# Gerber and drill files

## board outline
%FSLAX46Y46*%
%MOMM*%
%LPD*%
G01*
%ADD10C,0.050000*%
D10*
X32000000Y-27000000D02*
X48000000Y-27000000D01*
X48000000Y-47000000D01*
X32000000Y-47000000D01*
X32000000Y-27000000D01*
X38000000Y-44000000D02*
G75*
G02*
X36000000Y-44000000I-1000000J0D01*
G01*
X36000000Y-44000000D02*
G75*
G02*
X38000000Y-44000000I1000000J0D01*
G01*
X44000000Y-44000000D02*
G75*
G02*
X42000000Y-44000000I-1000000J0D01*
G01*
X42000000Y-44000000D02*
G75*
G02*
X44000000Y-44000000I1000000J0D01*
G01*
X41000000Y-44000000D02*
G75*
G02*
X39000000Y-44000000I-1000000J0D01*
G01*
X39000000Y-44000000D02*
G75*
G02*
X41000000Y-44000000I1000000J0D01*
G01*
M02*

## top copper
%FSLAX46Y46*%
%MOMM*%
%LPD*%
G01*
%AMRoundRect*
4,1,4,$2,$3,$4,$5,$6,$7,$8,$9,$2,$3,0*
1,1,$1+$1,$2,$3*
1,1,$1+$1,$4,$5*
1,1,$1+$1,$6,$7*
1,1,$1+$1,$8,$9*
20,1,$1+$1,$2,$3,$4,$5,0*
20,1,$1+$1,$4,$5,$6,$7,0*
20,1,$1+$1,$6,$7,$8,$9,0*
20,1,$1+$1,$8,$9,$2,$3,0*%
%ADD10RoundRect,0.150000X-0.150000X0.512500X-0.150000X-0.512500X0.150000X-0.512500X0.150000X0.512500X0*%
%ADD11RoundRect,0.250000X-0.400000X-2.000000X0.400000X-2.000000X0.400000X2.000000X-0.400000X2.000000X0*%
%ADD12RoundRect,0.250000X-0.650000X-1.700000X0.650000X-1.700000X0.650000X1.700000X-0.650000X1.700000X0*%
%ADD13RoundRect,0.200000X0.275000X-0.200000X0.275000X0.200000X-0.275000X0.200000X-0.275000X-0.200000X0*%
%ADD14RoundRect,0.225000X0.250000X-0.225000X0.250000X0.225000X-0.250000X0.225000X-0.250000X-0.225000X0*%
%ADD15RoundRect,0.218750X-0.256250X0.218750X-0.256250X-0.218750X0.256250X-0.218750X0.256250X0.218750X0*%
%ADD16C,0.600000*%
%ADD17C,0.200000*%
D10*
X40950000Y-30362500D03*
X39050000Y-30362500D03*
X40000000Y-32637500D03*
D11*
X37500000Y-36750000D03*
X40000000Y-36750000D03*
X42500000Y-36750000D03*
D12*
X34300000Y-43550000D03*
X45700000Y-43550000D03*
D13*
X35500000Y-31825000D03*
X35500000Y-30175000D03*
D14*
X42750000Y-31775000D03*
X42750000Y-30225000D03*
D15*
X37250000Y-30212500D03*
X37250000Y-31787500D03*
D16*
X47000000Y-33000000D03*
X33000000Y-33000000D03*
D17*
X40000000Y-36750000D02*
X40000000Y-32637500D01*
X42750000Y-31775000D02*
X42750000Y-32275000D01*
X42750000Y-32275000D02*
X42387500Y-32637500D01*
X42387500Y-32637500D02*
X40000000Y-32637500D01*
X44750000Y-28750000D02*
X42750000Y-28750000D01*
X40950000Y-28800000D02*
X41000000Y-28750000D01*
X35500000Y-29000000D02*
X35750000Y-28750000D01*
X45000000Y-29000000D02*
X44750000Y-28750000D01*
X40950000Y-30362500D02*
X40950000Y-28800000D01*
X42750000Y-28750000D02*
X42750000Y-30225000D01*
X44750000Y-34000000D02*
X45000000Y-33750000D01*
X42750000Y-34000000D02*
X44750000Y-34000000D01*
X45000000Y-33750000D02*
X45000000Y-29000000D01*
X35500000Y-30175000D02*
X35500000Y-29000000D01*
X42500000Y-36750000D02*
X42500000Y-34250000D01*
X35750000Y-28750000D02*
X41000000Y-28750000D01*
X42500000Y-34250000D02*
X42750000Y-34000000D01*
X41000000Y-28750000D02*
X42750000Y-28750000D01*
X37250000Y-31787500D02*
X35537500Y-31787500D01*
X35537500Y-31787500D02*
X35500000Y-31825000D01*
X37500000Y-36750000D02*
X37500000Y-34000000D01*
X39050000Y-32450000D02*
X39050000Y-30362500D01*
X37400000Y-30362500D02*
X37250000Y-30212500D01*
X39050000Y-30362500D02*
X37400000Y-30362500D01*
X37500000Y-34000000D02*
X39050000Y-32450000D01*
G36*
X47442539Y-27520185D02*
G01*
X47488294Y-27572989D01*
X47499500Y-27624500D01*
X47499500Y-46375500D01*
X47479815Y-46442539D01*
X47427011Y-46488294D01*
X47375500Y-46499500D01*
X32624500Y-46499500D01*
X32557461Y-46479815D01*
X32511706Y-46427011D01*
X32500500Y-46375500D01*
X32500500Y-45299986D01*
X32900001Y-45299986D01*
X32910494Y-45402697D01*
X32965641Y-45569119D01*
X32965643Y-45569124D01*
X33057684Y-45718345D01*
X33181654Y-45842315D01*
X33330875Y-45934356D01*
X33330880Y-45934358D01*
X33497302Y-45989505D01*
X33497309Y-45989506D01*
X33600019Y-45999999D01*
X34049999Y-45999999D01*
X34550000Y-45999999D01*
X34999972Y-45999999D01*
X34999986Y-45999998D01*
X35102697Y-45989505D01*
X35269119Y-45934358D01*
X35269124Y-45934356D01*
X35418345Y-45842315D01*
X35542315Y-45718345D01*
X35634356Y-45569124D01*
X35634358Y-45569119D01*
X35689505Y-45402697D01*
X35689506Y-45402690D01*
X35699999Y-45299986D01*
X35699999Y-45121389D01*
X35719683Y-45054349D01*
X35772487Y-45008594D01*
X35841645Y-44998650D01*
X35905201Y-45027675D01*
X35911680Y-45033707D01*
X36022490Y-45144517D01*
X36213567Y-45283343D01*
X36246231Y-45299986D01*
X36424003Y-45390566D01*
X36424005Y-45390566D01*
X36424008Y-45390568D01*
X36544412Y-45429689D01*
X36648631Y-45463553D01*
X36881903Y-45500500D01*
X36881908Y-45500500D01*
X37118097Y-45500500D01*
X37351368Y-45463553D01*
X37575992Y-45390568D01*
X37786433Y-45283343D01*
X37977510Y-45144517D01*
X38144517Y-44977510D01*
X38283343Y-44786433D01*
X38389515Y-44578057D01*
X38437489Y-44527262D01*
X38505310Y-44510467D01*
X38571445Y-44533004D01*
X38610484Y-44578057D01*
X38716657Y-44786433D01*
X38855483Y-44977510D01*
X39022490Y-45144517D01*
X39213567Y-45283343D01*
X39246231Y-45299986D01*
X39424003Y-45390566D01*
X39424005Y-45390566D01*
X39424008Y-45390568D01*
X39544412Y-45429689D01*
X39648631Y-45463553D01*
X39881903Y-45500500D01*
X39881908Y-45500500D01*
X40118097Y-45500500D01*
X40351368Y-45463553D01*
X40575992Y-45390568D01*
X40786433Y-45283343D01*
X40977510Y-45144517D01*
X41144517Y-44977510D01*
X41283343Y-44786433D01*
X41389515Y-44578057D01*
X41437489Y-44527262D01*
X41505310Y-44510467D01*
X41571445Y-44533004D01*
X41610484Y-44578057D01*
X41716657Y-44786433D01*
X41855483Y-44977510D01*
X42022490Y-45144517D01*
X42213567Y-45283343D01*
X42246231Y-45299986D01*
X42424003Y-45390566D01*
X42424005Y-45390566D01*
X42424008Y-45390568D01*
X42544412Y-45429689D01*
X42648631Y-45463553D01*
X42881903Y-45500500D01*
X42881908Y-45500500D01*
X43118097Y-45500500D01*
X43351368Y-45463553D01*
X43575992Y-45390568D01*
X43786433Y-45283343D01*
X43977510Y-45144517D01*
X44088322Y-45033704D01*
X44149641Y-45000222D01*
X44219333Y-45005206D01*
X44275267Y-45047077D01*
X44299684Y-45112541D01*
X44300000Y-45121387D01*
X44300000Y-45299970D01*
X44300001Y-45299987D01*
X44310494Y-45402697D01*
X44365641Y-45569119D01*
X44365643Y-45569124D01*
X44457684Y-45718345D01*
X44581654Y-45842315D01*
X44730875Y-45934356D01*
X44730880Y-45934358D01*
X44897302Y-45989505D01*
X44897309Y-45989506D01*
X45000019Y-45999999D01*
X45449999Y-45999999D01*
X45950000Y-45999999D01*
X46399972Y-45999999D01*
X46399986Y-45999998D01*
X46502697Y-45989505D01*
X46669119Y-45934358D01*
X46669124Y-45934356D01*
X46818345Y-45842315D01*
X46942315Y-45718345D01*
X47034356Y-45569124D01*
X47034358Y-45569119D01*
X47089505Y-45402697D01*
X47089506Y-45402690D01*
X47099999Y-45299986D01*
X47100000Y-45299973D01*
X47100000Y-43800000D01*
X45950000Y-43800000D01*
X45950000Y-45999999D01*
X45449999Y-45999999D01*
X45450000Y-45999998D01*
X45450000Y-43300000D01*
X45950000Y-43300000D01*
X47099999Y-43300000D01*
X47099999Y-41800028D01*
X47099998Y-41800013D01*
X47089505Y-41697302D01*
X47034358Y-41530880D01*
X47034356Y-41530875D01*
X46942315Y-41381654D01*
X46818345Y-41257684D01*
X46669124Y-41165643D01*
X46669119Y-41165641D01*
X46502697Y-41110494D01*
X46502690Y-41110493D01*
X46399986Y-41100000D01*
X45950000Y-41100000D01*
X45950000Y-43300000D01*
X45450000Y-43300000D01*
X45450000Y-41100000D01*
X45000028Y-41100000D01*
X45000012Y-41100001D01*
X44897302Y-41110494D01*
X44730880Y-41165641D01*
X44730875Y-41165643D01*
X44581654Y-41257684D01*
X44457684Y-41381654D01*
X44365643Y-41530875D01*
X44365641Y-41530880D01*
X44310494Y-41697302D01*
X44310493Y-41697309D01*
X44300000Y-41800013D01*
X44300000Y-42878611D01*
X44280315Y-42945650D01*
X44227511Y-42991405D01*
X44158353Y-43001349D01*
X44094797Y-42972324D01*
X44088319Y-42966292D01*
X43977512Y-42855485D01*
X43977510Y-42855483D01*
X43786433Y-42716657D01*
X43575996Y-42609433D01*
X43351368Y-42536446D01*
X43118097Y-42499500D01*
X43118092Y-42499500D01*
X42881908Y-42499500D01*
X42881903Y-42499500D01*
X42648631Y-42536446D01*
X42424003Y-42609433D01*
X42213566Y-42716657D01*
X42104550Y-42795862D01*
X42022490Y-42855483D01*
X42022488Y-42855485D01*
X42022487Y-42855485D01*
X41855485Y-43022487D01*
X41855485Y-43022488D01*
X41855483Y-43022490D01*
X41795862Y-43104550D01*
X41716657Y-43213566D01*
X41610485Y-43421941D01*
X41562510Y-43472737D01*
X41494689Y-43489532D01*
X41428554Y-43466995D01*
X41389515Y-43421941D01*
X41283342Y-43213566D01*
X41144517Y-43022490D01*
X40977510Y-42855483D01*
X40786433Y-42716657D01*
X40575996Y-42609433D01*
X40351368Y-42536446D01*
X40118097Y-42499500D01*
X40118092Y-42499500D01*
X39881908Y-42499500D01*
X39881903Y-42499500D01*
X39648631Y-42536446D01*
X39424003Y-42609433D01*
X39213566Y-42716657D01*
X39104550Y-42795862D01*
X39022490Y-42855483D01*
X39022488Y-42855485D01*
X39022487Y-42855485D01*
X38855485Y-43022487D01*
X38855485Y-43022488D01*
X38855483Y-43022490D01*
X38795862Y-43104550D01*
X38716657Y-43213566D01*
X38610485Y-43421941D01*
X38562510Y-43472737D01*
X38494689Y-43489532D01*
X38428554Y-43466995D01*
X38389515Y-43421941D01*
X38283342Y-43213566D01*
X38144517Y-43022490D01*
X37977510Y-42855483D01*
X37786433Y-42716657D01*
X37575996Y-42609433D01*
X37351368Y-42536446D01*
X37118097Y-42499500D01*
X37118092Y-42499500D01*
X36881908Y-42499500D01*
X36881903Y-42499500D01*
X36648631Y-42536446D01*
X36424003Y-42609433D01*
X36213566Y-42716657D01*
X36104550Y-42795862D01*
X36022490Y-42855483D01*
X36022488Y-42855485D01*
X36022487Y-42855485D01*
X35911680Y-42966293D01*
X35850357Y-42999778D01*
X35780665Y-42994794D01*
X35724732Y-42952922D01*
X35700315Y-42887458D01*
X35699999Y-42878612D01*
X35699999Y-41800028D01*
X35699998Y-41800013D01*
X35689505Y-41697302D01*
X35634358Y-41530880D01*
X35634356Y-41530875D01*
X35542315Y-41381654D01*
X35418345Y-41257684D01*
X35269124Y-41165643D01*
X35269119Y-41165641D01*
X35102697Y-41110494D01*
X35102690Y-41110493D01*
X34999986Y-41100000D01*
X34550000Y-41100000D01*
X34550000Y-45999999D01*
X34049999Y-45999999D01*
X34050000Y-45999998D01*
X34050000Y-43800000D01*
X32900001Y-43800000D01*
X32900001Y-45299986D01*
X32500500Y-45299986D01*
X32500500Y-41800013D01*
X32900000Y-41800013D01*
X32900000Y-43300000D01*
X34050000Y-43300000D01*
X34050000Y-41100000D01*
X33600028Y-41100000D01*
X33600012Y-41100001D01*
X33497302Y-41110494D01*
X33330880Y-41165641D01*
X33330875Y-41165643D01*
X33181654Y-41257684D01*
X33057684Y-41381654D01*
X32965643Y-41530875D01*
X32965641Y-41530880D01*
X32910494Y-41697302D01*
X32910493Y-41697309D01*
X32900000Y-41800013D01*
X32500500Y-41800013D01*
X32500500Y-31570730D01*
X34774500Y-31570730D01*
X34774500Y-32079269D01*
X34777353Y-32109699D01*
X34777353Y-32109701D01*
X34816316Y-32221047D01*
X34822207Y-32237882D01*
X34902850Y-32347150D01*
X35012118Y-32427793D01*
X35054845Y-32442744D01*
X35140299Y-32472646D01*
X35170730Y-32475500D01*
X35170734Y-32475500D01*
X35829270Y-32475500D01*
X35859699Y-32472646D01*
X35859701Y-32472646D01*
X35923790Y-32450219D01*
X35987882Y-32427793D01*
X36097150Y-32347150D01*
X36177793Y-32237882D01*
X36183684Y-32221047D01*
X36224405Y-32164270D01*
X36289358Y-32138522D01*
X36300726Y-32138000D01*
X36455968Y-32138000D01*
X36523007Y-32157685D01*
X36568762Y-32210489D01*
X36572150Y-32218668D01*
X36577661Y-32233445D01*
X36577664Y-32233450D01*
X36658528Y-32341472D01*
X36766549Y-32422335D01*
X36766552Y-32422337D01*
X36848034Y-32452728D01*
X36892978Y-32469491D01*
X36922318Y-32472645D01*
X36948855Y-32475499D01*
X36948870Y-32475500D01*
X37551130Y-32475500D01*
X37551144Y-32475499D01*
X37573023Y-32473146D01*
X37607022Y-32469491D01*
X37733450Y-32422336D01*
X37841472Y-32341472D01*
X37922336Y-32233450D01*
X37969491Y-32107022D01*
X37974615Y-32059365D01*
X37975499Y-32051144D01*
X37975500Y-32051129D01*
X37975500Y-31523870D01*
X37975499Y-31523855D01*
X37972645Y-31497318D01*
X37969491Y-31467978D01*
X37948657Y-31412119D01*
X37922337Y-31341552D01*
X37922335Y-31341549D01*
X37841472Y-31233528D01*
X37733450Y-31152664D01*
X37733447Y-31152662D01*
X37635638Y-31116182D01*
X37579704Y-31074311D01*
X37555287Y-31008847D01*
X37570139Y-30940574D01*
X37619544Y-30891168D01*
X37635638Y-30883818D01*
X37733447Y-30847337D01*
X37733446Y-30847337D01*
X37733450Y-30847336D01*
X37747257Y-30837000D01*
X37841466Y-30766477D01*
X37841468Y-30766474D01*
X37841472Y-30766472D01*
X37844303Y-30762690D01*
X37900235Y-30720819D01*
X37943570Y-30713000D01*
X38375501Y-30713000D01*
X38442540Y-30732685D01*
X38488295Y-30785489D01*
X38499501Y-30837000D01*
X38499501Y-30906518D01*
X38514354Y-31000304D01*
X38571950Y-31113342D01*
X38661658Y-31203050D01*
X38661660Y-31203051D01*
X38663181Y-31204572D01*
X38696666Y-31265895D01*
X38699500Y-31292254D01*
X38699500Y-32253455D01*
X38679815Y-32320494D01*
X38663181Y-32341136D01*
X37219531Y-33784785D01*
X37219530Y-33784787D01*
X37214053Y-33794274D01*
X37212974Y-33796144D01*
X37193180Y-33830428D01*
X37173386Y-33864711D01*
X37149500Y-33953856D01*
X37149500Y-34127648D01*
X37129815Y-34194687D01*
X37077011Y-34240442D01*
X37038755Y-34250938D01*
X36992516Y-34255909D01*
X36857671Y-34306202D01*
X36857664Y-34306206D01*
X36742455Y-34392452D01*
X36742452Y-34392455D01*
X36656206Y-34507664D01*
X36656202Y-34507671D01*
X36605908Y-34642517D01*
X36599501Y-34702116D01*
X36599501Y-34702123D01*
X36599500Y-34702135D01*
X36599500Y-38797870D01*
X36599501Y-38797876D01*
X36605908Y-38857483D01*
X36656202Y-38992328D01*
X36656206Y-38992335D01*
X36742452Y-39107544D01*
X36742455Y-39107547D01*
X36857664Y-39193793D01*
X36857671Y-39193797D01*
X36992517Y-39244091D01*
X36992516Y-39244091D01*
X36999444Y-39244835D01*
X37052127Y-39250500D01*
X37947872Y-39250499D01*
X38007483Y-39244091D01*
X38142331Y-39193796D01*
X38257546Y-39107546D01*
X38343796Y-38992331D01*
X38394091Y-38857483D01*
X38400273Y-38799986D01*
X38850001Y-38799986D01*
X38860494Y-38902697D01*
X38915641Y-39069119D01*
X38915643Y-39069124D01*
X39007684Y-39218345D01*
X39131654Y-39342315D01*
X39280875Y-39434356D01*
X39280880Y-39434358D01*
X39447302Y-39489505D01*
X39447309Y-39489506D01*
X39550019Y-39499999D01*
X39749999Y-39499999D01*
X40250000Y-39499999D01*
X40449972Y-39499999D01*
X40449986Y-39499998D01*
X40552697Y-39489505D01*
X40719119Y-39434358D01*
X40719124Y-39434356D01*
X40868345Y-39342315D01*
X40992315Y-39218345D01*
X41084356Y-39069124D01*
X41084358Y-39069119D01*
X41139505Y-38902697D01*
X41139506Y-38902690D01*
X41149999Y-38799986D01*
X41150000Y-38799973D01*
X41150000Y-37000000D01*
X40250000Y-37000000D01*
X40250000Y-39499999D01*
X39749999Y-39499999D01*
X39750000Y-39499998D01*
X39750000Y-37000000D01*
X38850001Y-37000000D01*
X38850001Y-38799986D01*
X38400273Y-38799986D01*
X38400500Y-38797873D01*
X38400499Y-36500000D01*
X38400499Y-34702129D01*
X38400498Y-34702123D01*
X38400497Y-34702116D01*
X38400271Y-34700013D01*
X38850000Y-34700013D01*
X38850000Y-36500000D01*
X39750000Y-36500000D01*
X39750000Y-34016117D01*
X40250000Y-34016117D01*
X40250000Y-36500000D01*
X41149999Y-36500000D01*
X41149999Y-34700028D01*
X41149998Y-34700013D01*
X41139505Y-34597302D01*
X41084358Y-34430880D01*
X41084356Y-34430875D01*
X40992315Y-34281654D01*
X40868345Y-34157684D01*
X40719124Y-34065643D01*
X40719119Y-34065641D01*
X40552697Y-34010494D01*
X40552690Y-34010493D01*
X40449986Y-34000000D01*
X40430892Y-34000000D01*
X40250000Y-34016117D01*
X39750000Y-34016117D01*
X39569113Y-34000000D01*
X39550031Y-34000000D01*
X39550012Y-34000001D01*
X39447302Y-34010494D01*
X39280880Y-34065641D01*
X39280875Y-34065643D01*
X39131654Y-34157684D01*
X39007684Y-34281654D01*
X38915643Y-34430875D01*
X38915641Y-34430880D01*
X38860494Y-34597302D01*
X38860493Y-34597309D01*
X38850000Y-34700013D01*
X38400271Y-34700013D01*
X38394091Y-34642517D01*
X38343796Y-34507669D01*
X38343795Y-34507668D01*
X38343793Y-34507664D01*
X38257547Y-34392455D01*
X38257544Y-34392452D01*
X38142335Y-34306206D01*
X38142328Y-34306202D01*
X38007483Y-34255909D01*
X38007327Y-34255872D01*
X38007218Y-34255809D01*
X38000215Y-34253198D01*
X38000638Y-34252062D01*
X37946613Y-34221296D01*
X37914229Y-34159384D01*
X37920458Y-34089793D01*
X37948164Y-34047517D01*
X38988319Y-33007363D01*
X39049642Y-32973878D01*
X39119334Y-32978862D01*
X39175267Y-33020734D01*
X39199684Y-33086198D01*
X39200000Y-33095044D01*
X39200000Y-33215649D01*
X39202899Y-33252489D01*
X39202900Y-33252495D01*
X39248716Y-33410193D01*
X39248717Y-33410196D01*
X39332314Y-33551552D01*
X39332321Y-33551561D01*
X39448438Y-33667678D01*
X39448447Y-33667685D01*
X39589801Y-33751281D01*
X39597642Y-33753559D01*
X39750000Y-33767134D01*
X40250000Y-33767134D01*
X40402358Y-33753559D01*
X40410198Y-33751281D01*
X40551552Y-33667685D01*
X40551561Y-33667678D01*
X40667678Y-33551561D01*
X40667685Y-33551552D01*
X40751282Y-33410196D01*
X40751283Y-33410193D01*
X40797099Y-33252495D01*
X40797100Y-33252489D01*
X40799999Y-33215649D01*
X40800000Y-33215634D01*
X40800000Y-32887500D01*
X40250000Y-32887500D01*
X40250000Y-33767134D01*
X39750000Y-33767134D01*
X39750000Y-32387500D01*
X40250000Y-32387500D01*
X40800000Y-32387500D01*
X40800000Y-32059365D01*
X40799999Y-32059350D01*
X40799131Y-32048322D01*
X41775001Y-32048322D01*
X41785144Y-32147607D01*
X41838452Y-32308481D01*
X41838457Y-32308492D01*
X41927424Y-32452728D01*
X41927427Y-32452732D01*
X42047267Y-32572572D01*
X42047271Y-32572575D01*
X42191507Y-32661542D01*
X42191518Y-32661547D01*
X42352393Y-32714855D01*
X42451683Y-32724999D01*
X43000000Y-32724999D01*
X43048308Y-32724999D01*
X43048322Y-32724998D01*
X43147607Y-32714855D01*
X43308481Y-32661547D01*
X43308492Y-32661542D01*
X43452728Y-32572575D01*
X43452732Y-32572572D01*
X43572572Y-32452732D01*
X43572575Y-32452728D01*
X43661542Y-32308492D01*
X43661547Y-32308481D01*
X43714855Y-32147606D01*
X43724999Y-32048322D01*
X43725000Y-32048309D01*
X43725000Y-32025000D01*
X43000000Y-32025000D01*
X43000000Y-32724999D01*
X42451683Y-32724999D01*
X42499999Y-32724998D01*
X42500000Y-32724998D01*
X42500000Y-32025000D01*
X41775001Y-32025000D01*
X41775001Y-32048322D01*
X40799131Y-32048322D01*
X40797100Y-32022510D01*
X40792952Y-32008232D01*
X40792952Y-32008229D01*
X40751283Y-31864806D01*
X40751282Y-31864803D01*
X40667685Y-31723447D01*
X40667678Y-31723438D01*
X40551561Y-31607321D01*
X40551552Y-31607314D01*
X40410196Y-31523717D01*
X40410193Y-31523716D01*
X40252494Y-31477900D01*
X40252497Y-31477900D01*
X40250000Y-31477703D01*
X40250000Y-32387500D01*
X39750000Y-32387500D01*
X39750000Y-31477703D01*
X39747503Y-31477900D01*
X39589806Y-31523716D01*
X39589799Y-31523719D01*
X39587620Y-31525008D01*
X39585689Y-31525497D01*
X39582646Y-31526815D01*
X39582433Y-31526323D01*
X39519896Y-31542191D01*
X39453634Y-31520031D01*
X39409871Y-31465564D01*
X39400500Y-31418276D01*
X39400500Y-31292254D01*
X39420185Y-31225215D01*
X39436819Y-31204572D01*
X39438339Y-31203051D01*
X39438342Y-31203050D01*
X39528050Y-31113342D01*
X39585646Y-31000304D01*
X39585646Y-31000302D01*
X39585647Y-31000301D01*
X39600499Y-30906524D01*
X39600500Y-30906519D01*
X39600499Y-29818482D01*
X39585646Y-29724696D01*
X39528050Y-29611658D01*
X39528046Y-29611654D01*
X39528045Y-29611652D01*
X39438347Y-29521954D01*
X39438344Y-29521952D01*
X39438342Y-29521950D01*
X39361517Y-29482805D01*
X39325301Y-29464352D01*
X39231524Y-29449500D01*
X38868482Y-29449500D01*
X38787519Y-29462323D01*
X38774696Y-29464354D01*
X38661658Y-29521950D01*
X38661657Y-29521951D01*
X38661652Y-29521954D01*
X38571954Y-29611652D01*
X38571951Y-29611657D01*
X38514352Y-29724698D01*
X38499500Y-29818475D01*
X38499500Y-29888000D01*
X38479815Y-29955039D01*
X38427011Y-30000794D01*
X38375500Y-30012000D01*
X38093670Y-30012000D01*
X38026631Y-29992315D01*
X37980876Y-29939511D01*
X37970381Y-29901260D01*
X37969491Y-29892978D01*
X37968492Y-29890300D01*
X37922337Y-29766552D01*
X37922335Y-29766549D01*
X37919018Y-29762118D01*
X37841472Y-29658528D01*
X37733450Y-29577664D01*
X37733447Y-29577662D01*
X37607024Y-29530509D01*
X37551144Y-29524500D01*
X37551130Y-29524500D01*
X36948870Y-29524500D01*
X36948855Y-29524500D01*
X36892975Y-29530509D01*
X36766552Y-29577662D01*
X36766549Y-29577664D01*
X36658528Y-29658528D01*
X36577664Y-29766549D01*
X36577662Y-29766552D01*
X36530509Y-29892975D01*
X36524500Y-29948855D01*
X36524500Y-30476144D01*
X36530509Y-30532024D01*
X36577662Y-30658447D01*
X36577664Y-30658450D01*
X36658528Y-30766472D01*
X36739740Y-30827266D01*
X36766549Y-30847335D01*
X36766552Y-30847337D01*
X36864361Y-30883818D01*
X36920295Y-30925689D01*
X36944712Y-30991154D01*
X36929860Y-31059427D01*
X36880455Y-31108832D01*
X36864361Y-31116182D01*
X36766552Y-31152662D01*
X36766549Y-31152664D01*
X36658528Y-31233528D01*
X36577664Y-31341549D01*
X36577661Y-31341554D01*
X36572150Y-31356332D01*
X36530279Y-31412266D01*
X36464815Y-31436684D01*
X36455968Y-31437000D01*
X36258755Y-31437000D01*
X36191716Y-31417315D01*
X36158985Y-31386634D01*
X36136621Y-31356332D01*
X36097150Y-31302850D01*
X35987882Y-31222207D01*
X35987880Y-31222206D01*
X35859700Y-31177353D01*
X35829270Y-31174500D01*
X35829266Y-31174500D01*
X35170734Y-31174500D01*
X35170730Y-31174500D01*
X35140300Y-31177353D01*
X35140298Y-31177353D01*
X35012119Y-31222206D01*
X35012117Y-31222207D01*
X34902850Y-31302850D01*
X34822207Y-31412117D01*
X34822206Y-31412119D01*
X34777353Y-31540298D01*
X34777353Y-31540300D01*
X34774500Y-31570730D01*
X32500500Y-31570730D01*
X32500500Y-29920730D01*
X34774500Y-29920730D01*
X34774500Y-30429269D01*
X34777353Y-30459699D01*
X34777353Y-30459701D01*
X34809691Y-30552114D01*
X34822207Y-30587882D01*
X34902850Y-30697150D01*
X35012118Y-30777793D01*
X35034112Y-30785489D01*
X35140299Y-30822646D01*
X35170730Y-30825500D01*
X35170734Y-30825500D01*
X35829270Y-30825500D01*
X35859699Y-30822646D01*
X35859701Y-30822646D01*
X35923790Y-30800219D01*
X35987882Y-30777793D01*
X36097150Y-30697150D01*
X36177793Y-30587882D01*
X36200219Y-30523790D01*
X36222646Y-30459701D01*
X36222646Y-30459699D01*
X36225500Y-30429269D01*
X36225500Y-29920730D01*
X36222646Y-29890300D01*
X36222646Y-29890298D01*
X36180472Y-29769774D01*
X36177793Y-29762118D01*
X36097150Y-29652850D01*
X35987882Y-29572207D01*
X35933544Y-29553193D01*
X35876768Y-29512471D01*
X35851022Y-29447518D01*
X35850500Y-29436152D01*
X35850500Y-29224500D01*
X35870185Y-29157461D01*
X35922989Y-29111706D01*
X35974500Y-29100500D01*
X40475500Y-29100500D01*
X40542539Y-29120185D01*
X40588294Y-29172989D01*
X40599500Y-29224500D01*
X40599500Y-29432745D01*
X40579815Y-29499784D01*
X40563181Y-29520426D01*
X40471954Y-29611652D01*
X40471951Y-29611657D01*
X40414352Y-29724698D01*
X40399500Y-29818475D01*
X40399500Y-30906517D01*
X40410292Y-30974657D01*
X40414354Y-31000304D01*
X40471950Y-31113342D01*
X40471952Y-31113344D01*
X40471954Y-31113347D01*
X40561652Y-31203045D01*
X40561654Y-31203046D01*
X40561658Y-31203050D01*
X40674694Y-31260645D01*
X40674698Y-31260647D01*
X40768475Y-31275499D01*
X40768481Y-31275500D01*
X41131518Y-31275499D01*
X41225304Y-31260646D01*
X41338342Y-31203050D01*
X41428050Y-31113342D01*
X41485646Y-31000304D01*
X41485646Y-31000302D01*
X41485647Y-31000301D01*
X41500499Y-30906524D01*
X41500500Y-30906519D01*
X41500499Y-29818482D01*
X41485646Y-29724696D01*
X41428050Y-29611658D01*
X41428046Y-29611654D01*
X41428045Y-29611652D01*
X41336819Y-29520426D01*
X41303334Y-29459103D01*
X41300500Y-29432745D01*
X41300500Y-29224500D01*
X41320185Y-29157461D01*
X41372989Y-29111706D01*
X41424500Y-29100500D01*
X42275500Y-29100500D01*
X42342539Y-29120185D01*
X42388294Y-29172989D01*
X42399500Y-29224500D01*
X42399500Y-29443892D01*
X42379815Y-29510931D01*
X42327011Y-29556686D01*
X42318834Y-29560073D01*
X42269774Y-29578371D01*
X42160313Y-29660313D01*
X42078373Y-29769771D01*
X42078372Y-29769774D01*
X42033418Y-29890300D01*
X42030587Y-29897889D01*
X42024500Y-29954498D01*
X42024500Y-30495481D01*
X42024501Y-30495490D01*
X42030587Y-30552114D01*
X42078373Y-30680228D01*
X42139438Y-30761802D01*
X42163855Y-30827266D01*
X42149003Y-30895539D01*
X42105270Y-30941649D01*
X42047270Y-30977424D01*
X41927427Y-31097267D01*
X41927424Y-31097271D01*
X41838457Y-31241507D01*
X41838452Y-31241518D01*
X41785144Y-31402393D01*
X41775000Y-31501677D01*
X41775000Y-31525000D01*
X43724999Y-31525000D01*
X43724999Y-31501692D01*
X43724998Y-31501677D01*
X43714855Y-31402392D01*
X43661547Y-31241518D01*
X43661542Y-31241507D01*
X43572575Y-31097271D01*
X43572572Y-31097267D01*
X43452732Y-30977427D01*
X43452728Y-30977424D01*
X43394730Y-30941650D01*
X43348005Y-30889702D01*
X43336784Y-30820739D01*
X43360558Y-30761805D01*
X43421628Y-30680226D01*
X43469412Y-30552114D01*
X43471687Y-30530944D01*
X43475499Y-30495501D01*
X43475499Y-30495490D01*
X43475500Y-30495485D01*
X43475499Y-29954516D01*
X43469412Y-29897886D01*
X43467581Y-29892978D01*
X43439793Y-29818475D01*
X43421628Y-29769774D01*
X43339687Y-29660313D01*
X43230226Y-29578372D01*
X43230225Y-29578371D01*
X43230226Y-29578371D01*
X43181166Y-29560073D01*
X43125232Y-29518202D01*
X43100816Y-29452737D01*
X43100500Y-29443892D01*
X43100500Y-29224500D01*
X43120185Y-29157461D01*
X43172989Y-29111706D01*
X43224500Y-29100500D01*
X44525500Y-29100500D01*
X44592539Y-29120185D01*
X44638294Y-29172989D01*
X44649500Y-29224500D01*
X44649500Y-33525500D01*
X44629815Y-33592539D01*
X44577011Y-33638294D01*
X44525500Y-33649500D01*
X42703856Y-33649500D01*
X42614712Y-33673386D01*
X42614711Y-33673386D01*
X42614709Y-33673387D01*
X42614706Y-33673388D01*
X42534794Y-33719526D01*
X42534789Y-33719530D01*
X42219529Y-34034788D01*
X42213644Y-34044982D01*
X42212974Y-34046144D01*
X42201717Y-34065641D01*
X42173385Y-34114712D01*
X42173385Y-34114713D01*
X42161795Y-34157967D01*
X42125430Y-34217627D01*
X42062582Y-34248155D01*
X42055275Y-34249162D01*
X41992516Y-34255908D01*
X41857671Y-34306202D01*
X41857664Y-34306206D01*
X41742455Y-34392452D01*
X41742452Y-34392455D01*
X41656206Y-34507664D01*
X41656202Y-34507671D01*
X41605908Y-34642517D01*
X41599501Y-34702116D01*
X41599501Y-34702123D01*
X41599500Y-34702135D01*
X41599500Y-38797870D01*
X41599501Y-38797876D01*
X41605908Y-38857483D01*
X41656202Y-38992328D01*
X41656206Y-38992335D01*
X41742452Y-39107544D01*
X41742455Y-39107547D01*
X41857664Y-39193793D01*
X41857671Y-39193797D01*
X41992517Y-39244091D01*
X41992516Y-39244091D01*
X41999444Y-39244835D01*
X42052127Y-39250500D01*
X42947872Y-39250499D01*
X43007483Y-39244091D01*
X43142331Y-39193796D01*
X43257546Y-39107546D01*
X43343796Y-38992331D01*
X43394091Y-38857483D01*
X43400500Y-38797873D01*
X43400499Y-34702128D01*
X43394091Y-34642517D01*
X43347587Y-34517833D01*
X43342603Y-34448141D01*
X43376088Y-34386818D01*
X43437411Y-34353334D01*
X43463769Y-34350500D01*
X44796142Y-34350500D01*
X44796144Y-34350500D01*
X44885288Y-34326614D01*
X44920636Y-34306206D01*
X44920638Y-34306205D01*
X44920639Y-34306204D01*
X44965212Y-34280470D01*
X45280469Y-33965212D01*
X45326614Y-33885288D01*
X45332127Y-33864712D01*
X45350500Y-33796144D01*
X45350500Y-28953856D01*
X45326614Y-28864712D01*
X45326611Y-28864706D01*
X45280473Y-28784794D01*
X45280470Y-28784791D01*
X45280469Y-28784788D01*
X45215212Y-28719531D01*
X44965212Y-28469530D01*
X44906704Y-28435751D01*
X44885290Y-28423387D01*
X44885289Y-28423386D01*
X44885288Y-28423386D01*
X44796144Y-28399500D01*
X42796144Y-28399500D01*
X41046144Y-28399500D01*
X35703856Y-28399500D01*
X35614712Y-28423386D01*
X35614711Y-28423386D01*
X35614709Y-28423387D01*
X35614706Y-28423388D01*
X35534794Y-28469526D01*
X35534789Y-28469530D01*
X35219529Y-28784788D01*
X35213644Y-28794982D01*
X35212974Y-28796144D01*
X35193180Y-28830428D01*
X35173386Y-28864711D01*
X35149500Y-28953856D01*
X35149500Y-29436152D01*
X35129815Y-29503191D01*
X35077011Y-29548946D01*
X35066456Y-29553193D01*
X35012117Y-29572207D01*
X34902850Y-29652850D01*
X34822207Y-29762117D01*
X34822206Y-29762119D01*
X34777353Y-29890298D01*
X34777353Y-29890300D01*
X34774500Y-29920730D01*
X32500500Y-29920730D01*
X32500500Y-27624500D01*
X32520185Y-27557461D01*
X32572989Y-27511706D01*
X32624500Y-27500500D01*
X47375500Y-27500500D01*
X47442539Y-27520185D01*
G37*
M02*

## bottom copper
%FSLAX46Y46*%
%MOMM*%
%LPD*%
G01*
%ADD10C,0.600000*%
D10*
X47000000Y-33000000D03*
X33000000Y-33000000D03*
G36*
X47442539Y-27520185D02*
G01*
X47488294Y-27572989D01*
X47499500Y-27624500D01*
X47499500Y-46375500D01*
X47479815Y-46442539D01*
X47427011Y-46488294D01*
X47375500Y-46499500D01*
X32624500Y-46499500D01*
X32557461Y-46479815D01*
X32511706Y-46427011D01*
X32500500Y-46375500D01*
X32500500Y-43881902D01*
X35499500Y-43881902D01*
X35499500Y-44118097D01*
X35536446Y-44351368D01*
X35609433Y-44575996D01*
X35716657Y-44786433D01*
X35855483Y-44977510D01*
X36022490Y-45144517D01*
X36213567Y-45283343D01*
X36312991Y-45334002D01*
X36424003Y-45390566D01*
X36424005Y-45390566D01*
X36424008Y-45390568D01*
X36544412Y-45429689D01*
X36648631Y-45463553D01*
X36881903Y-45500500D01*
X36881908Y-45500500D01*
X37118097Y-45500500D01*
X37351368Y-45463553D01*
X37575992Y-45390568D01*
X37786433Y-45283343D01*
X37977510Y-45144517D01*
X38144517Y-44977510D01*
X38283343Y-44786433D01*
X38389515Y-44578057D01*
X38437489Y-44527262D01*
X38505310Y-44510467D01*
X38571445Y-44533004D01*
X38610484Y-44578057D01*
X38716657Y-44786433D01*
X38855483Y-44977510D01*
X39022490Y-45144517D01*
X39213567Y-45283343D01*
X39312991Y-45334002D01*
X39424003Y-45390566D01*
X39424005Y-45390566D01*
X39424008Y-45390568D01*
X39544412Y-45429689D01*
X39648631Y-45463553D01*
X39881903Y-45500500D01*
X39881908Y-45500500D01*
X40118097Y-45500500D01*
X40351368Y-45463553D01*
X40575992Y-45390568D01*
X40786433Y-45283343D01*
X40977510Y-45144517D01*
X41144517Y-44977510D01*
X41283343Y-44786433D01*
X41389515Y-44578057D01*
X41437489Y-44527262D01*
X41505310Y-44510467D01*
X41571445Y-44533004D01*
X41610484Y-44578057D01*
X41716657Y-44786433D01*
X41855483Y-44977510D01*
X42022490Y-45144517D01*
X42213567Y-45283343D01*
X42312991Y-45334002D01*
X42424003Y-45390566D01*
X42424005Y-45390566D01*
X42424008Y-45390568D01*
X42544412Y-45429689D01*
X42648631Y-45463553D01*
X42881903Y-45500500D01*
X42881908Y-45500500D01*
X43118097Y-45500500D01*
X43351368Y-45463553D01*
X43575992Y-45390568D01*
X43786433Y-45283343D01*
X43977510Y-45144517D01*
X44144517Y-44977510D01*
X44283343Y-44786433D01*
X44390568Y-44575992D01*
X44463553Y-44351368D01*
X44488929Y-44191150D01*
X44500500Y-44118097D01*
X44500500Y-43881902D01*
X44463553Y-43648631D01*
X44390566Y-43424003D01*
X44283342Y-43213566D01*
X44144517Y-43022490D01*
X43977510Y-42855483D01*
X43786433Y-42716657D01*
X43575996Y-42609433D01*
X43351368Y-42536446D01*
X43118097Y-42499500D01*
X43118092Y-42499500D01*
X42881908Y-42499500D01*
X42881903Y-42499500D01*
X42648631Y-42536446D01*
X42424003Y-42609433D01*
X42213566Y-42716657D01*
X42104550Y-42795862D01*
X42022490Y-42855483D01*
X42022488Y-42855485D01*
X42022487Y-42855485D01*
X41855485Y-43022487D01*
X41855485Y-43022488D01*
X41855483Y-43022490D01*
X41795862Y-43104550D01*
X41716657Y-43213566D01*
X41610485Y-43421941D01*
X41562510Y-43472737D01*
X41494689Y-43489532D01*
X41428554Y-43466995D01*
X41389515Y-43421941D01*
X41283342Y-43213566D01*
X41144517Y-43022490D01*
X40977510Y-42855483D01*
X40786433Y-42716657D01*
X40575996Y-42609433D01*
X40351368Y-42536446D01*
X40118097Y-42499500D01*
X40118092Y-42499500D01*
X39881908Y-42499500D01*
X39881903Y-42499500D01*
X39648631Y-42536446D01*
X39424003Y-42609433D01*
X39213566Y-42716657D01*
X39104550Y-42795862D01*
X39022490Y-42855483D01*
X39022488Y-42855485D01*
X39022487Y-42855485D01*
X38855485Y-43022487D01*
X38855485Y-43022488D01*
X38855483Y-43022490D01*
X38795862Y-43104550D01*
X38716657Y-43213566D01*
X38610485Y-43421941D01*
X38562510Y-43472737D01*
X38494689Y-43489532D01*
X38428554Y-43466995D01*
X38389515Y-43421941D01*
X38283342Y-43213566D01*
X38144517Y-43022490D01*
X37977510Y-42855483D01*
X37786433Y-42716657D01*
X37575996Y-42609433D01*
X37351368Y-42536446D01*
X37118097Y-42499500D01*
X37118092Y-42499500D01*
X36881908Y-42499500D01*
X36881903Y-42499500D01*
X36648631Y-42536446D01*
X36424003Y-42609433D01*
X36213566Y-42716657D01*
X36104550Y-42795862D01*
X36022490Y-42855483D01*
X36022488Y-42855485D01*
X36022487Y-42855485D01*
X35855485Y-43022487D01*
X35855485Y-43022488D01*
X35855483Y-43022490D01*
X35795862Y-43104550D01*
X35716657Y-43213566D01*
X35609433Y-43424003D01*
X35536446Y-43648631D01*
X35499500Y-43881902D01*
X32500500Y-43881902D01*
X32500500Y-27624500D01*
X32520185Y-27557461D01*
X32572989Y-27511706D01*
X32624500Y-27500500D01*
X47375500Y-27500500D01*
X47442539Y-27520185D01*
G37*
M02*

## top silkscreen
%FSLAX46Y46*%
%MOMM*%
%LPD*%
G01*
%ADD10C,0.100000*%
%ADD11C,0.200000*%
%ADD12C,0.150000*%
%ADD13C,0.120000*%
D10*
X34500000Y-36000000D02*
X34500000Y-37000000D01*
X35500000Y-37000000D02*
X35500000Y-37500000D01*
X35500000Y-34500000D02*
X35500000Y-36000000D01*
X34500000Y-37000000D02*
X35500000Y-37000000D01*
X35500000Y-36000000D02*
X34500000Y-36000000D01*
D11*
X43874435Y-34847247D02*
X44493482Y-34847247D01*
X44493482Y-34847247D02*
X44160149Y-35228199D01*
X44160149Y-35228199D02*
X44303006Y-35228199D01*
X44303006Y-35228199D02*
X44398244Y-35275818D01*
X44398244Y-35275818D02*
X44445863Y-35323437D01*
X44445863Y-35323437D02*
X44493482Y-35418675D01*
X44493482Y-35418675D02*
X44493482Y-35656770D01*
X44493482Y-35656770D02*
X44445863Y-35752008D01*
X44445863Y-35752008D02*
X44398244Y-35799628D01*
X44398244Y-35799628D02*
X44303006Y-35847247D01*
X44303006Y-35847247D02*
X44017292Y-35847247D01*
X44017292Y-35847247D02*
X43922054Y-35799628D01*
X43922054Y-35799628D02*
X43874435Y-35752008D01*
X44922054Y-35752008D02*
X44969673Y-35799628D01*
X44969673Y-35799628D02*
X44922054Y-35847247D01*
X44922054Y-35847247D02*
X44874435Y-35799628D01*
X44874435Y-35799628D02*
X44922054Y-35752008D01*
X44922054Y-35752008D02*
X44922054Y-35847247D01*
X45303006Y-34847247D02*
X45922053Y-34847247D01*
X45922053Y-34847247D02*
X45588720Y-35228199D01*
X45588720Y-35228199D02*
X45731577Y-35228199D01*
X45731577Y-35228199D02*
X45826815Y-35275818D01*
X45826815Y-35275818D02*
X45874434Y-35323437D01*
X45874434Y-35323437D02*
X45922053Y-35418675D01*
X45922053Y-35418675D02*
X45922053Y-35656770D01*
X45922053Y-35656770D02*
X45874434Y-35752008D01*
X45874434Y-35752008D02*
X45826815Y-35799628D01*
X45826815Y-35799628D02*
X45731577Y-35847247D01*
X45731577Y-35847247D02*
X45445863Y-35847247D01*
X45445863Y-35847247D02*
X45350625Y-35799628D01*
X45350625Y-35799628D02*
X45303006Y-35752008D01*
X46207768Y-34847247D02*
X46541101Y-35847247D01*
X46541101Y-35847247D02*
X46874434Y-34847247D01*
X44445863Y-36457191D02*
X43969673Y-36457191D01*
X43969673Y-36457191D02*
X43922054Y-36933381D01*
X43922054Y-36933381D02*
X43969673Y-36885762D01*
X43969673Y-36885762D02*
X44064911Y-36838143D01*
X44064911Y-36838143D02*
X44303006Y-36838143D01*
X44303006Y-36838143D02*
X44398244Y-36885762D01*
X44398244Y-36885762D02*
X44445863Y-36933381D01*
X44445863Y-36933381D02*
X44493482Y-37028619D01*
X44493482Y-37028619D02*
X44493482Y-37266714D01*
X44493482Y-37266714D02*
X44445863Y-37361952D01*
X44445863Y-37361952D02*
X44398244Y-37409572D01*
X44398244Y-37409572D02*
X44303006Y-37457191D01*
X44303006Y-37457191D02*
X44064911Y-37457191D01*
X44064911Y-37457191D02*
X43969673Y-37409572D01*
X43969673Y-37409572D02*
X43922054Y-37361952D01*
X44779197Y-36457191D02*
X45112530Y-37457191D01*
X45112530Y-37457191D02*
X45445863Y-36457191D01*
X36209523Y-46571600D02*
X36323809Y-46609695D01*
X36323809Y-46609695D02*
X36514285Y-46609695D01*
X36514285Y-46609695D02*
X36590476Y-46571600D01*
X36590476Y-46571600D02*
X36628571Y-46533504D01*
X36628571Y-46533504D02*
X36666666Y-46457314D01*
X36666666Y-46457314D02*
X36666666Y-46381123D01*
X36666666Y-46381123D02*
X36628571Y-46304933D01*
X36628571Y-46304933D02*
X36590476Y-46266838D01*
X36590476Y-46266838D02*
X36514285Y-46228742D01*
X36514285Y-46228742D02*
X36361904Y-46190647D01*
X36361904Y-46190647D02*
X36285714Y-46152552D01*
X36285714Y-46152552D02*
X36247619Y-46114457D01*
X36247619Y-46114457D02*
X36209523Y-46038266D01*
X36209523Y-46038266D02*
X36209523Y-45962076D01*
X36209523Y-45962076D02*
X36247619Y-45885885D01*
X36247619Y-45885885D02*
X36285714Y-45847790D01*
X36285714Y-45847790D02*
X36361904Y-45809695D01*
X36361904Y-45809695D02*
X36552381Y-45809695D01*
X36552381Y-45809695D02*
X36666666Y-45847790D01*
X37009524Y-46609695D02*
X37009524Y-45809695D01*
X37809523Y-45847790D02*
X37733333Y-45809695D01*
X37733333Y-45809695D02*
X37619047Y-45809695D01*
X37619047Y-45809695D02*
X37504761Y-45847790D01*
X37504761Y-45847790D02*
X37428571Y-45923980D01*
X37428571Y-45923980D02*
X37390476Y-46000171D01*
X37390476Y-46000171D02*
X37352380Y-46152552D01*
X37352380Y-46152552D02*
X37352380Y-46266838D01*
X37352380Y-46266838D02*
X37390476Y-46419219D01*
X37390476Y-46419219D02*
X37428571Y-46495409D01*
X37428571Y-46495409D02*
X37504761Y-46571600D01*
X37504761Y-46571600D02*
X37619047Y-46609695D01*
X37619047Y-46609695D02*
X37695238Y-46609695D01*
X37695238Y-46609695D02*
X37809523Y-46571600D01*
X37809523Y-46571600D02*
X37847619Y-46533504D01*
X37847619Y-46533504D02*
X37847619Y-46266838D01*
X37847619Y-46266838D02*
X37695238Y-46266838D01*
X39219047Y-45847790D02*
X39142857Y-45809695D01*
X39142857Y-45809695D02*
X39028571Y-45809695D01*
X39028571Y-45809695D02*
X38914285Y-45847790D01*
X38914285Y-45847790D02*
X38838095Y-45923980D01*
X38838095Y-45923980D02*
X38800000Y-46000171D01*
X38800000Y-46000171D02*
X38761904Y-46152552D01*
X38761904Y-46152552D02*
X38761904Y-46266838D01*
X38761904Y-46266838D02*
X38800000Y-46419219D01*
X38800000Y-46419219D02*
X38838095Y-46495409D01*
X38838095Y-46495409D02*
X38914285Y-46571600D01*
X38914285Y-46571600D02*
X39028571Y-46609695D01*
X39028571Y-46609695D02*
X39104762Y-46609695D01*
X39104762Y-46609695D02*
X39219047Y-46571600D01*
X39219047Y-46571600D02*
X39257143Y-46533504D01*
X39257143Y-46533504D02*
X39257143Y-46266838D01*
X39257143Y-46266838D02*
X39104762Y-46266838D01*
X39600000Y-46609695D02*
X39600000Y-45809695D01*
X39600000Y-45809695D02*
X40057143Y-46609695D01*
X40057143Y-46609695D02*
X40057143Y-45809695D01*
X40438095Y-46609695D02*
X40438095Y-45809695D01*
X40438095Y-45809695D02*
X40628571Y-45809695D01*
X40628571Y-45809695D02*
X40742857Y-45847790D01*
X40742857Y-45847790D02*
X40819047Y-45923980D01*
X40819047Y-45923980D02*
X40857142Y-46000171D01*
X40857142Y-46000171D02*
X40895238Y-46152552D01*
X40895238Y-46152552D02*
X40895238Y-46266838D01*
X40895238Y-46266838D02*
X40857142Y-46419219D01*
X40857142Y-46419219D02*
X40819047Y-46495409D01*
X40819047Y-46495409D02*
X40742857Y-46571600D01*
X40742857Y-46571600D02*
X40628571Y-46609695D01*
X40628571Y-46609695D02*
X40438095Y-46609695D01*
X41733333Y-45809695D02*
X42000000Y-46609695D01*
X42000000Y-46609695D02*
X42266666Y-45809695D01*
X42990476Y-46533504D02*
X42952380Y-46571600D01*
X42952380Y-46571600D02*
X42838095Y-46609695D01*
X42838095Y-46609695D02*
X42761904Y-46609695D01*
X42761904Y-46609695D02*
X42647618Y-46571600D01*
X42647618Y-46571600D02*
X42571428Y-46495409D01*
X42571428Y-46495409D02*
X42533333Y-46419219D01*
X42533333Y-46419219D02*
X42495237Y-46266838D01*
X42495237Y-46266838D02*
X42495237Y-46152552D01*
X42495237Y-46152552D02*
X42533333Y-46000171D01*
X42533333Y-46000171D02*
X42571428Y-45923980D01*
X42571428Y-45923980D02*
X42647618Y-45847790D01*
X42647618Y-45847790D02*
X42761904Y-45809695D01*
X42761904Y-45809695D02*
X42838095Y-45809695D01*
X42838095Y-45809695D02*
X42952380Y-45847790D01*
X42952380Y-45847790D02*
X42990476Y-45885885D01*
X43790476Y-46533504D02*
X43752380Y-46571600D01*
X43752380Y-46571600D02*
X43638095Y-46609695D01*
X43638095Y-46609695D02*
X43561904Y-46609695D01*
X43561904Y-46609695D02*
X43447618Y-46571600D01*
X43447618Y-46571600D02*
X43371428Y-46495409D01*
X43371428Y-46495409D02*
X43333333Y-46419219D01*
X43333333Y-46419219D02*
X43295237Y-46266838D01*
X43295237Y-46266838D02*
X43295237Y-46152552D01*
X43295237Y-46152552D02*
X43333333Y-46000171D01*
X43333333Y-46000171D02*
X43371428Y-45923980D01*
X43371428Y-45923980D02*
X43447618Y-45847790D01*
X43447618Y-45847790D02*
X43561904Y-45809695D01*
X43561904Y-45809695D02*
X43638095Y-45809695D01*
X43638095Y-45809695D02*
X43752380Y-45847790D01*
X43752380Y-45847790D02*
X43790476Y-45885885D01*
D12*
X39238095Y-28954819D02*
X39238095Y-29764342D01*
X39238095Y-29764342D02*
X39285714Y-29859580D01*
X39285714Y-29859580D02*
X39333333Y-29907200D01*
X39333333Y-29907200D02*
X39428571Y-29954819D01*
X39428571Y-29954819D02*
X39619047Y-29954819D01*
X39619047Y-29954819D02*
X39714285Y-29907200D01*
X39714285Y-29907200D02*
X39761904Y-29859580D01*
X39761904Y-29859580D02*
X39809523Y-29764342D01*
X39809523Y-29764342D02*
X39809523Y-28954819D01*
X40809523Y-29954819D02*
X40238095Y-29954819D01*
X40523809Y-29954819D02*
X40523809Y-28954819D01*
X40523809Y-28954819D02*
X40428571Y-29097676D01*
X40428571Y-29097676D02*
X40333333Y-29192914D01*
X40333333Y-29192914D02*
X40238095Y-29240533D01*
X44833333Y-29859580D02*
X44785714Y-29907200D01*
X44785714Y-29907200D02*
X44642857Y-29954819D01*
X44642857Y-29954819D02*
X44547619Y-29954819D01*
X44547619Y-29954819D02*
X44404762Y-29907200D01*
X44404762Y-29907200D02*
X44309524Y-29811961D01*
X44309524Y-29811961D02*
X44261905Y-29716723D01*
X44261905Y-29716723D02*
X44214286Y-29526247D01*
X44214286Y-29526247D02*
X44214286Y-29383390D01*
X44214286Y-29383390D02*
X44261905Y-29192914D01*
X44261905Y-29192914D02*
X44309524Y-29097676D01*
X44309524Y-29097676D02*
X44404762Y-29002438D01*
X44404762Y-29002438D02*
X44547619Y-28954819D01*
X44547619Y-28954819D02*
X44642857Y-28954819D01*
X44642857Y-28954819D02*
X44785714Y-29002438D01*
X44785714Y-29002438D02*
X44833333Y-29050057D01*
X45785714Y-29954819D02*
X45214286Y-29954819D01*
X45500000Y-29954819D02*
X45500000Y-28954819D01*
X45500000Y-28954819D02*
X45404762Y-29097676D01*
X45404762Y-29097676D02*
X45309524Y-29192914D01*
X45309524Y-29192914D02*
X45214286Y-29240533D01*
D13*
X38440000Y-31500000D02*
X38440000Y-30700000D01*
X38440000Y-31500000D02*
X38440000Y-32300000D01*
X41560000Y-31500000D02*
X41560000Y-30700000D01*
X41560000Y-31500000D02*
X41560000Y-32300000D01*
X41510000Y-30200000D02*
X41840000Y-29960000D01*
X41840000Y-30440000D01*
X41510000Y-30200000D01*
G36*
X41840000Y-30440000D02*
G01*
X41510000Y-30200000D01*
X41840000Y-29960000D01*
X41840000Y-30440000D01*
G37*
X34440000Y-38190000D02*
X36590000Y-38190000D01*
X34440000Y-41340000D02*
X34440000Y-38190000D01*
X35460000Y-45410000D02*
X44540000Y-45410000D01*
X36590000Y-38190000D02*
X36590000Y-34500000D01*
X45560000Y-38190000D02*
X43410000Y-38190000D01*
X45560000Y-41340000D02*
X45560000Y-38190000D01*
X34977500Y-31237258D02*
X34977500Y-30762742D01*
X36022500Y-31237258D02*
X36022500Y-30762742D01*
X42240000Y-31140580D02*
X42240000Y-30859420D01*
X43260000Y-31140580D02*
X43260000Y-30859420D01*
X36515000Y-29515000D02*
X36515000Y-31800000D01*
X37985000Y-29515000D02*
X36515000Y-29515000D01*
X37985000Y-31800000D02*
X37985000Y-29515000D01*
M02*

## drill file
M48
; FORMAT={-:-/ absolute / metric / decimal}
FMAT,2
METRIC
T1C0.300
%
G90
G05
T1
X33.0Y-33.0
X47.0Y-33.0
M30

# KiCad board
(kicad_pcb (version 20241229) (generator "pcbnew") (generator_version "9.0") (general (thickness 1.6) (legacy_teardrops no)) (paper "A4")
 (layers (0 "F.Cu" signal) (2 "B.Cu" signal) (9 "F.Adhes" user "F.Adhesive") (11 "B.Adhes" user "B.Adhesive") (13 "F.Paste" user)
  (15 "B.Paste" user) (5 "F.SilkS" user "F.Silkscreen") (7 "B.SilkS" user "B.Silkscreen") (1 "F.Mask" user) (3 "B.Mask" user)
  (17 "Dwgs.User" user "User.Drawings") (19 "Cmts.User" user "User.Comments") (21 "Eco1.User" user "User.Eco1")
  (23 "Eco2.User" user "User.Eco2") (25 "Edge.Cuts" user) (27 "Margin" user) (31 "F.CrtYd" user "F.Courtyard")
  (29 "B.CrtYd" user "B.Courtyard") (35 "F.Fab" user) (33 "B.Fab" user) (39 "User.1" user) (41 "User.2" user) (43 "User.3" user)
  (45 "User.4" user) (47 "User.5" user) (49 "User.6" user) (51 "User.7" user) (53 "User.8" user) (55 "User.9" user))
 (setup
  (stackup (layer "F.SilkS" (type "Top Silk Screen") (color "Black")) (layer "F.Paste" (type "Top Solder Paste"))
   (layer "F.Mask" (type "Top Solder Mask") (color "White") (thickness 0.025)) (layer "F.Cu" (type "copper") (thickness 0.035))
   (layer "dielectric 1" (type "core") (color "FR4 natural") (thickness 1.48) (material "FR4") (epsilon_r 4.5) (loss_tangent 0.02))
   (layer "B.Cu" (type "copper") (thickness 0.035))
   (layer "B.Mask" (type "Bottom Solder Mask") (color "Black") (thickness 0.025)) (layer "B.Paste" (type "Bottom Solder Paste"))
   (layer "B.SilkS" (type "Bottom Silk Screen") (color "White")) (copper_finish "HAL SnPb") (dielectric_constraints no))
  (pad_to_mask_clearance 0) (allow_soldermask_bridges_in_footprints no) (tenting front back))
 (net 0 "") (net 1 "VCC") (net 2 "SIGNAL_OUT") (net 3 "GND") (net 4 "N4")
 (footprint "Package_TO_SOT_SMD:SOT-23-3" (layer "F.Cu") (at 40 31.5 -90)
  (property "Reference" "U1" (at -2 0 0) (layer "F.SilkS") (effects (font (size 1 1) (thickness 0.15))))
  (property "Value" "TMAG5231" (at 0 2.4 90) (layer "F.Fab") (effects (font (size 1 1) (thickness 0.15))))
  (fp_line (start 0 1.56) (end -0.8 1.56) (stroke (width 0.12) (type solid)) (layer "F.SilkS"))
  (fp_line (start 0 1.56) (end 0.8 1.56) (stroke (width 0.12) (type solid)) (layer "F.SilkS"))
  (fp_line (start 0 -1.56) (end -0.8 -1.56) (stroke (width 0.12) (type solid)) (layer "F.SilkS"))
  (fp_line (start 0 -1.56) (end 0.8 -1.56) (stroke (width 0.12) (type solid)) (layer "F.SilkS"))
  (fp_poly
   (pts (xy -1.3 -1.51) (xy -1.54 -1.84) (xy -1.06 -1.84) (xy -1.3 -1.51)) (stroke (width 0.12) (type solid)) (fill yes) (layer "F.SilkS"))
  (pad "1" smd roundrect (at -1.1375 -0.95 270) (size 1.325 0.6) (layers "F.Cu" "F.Mask" "F.Paste") (roundrect_rratio 0.25) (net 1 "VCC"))
  (pad "2" smd roundrect (at -1.1375 0.95 270) (size 1.325 0.6) (layers "F.Cu" "F.Mask" "F.Paste") (roundrect_rratio 0.25)
   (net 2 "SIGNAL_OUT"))
  (pad "3" smd roundrect (at 1.1375 0 270) (size 1.325 0.6) (layers "F.Cu" "F.Mask" "F.Paste") (roundrect_rratio 0.25) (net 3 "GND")))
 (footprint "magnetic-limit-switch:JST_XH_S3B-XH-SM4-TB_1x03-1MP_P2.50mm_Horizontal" (layer "F.Cu") (at 40 40)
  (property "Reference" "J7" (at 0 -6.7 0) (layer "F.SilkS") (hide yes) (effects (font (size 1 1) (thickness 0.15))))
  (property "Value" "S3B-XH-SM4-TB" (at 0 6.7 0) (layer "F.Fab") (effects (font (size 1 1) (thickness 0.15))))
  (fp_line (start -5.56 -1.81) (end -3.41 -1.81) (stroke (width 0.12) (type solid)) (layer "F.SilkS"))
  (fp_line (start -5.56 1.34) (end -5.56 -1.81) (stroke (width 0.12) (type solid)) (layer "F.SilkS"))
  (fp_line (start -4.54 5.41) (end 4.54 5.41) (stroke (width 0.12) (type solid)) (layer "F.SilkS"))
  (fp_line (start -3.41 -1.81) (end -3.41 -5.5) (stroke (width 0.12) (type solid)) (layer "F.SilkS"))
  (fp_line (start 5.56 -1.81) (end 3.41 -1.81) (stroke (width 0.12) (type solid)) (layer "F.SilkS"))
  (fp_line (start 5.56 1.34) (end 5.56 -1.81) (stroke (width 0.12) (type solid)) (layer "F.SilkS"))
  (pad "1" smd roundrect (at -2.5 -3.25) (size 1.3 4.5) (layers "F.Cu" "F.Mask" "F.Paste") (roundrect_rratio 0.192308) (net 2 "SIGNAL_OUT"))
  (pad "2" smd roundrect (at 0 -3.25) (size 1.3 4.5) (layers "F.Cu" "F.Mask" "F.Paste") (roundrect_rratio 0.192308) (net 3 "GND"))
  (pad "3" smd roundrect (at 2.5 -3.25) (size 1.3 4.5) (layers "F.Cu" "F.Mask" "F.Paste") (roundrect_rratio 0.192308) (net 1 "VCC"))
  (pad "MP" smd roundrect (at -5.7 3.55) (size 1.8 3.9) (layers "F.Cu" "F.Mask" "F.Paste") (roundrect_rratio 0.138889) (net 3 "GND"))
  (pad "MP" smd roundrect (at 5.7 3.55) (size 1.8 3.9) (layers "F.Cu" "F.Mask" "F.Paste") (roundrect_rratio 0.138889) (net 3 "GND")))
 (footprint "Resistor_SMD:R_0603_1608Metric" (layer "F.Cu") (at 35.5 31 90)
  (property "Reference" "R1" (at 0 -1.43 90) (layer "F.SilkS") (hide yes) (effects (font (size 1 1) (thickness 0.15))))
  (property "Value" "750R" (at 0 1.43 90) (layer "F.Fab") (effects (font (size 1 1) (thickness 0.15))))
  (fp_line (start -0.237258 -0.5225) (end 0.237258 -0.5225) (stroke (width 0.12) (type solid)) (layer "F.SilkS"))
  (fp_line (start -0.237258 0.5225) (end 0.237258 0.5225) (stroke (width 0.12) (type solid)) (layer "F.SilkS"))
  (pad "1" smd roundrect (at -0.825 0 90) (size 0.8 0.95) (layers "F.Cu" "F.Mask" "F.Paste") (roundrect_rratio 0.25) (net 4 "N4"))
  (pad "2" smd roundrect (at 0.825 0 90) (size 0.8 0.95) (layers "F.Cu" "F.Mask" "F.Paste") (roundrect_rratio 0.25) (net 1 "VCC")))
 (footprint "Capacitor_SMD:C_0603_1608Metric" (layer "F.Cu") (at 42.75 31 90)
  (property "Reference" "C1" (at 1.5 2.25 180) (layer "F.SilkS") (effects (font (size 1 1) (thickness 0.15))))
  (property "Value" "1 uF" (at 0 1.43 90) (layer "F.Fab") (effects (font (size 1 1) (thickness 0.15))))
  (fp_line (start -0.14058 -0.51) (end 0.14058 -0.51) (stroke (width 0.12) (type solid)) (layer "F.SilkS"))
  (fp_line (start -0.14058 0.51) (end 0.14058 0.51) (stroke (width 0.12) (type solid)) (layer "F.SilkS"))
  (pad "1" smd roundrect (at -0.775 0 90) (size 0.9 0.95) (layers "F.Cu" "F.Mask" "F.Paste") (roundrect_rratio 0.25) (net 3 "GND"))
  (pad "2" smd roundrect (at 0.775 0 90) (size 0.9 0.95) (layers "F.Cu" "F.Mask" "F.Paste") (roundrect_rratio 0.25) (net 1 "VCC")))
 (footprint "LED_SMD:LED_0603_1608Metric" (layer "F.Cu") (at 37.25 31 -90)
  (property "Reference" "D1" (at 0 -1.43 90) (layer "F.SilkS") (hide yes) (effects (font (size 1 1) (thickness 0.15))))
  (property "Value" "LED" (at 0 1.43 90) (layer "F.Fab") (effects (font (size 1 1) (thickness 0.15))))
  (fp_line (start -1.485 0.735) (end 0.8 0.735) (stroke (width 0.12) (type solid)) (layer "F.SilkS"))
  (fp_line (start -1.485 -0.735) (end -1.485 0.735) (stroke (width 0.12) (type solid)) (layer "F.SilkS"))
  (fp_line (start 0.8 -0.735) (end -1.485 -0.735) (stroke (width 0.12) (type solid)) (layer "F.SilkS"))
  (pad "1" smd roundrect (at -0.7875 0 270) (size 0.875 0.95) (layers "F.Cu" "F.Mask" "F.Paste") (roundrect_rratio 0.25)
   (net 2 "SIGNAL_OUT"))
  (pad "2" smd roundrect (at 0.7875 0 270) (size 0.875 0.95) (layers "F.Cu" "F.Mask" "F.Paste") (roundrect_rratio 0.25) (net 4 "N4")))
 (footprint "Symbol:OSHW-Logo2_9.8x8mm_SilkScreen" (layer "B.Cu") (at 40.5 34 90)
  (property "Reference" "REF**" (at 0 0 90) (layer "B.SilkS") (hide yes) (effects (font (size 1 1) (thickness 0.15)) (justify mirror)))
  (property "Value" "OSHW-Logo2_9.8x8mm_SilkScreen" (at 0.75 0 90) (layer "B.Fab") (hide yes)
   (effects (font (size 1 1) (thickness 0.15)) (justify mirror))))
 (gr_line (start 34.5 36) (end 34.5 37) (stroke (width 0.1) (type default)) (layer "F.SilkS"))
 (gr_line (start 35.5 37) (end 35.5 37.5) (stroke (width 0.1) (type default)) (layer "F.SilkS"))
 (gr_line (start 35.5 34.5) (end 35.5 36) (stroke (width 0.1) (type default)) (layer "F.SilkS"))
 (gr_line (start 34.5 37) (end 35.5 37) (stroke (width 0.1) (type default)) (layer "F.SilkS"))
 (gr_line (start 35.5 36) (end 34.5 36) (stroke (width 0.1) (type default)) (layer "F.SilkS"))
 (gr_rect (start 32 27) (end 48 47) (stroke (width 0.05) (type default)) (fill no) (layer "Edge.Cuts"))
 (gr_circle (center 37 44) (end 38 44) (stroke (width 0.05) (type solid)) (fill no) (layer "Edge.Cuts"))
 (gr_circle (center 43 44) (end 44 44) (stroke (width 0.05) (type solid)) (fill no) (layer "Edge.Cuts"))
 (gr_circle (center 40 44) (end 41 44) (stroke (width 0.05) (type solid)) (fill no) (layer "Edge.Cuts"))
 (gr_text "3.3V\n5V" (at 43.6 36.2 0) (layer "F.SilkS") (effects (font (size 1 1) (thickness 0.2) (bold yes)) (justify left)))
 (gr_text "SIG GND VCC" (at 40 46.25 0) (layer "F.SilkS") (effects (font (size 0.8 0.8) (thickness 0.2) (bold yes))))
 (segment (start 40 36.75) (end 40 32.6375) (width 0.2) (layer "F.Cu") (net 3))
 (segment (start 42.75 31.775) (end 42.75 32.275) (width 0.2) (layer "F.Cu") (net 3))
 (segment (start 42.75 32.275) (end 42.3875 32.6375) (width 0.2) (layer "F.Cu") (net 3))
 (segment (start 42.3875 32.6375) (end 40 32.6375) (width 0.2) (layer "F.Cu") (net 3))
 (via (at 47 33) (size 0.6) (drill 0.3) (layers "F.Cu" "B.Cu") (free yes) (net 3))
 (via (at 33 33) (size 0.6) (drill 0.3) (layers "F.Cu" "B.Cu") (free yes) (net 3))
 (segment (start 44.75 28.75) (end 42.75 28.75) (width 0.2) (layer "F.Cu") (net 1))
 (segment (start 40.95 28.8) (end 41 28.75) (width 0.2) (layer "F.Cu") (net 1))
 (segment (start 35.5 29) (end 35.75 28.75) (width 0.2) (layer "F.Cu") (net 1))
 (segment (start 45 29) (end 44.75 28.75) (width 0.2) (layer "F.Cu") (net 1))
 (segment (start 40.95 30.3625) (end 40.95 28.8) (width 0.2) (layer "F.Cu") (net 1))
 (segment (start 42.75 28.75) (end 42.75 30.225) (width 0.2) (layer "F.Cu") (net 1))
 (segment (start 44.75 34) (end 45 33.75) (width 0.2) (layer "F.Cu") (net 1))
 (segment (start 42.75 34) (end 44.75 34) (width 0.2) (layer "F.Cu") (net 1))
 (segment (start 45 33.75) (end 45 29) (width 0.2) (layer "F.Cu") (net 1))
 (segment (start 35.5 30.175) (end 35.5 29) (width 0.2) (layer "F.Cu") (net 1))
 (segment (start 42.5 36.75) (end 42.5 34.25) (width 0.2) (layer "F.Cu") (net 1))
 (segment (start 35.75 28.75) (end 41 28.75) (width 0.2) (layer "F.Cu") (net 1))
 (segment (start 42.5 34.25) (end 42.75 34) (width 0.2) (layer "F.Cu") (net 1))
 (segment (start 41 28.75) (end 42.75 28.75) (width 0.2) (layer "F.Cu") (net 1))
 (segment (start 37.25 31.7875) (end 35.5375 31.7875) (width 0.2) (layer "F.Cu") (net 4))
 (segment (start 35.5375 31.7875) (end 35.5 31.825) (width 0.2) (layer "F.Cu") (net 4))
 (segment (start 37.5 36.75) (end 37.5 34) (width 0.2) (layer "F.Cu") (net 2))
 (segment (start 39.05 32.45) (end 39.05 30.3625) (width 0.2) (layer "F.Cu") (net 2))
 (segment (start 37.4 30.3625) (end 37.25 30.2125) (width 0.2) (layer "F.Cu") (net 2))
 (segment (start 39.05 30.3625) (end 37.4 30.3625) (width 0.2) (layer "F.Cu") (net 2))
 (segment (start 37.5 34) (end 39.05 32.45) (width 0.2) (layer "F.Cu") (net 2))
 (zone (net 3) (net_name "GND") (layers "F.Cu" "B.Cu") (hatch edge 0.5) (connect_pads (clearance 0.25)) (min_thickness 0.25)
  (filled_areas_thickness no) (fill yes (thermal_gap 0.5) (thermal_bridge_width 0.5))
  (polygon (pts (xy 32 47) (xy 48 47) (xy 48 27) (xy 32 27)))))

